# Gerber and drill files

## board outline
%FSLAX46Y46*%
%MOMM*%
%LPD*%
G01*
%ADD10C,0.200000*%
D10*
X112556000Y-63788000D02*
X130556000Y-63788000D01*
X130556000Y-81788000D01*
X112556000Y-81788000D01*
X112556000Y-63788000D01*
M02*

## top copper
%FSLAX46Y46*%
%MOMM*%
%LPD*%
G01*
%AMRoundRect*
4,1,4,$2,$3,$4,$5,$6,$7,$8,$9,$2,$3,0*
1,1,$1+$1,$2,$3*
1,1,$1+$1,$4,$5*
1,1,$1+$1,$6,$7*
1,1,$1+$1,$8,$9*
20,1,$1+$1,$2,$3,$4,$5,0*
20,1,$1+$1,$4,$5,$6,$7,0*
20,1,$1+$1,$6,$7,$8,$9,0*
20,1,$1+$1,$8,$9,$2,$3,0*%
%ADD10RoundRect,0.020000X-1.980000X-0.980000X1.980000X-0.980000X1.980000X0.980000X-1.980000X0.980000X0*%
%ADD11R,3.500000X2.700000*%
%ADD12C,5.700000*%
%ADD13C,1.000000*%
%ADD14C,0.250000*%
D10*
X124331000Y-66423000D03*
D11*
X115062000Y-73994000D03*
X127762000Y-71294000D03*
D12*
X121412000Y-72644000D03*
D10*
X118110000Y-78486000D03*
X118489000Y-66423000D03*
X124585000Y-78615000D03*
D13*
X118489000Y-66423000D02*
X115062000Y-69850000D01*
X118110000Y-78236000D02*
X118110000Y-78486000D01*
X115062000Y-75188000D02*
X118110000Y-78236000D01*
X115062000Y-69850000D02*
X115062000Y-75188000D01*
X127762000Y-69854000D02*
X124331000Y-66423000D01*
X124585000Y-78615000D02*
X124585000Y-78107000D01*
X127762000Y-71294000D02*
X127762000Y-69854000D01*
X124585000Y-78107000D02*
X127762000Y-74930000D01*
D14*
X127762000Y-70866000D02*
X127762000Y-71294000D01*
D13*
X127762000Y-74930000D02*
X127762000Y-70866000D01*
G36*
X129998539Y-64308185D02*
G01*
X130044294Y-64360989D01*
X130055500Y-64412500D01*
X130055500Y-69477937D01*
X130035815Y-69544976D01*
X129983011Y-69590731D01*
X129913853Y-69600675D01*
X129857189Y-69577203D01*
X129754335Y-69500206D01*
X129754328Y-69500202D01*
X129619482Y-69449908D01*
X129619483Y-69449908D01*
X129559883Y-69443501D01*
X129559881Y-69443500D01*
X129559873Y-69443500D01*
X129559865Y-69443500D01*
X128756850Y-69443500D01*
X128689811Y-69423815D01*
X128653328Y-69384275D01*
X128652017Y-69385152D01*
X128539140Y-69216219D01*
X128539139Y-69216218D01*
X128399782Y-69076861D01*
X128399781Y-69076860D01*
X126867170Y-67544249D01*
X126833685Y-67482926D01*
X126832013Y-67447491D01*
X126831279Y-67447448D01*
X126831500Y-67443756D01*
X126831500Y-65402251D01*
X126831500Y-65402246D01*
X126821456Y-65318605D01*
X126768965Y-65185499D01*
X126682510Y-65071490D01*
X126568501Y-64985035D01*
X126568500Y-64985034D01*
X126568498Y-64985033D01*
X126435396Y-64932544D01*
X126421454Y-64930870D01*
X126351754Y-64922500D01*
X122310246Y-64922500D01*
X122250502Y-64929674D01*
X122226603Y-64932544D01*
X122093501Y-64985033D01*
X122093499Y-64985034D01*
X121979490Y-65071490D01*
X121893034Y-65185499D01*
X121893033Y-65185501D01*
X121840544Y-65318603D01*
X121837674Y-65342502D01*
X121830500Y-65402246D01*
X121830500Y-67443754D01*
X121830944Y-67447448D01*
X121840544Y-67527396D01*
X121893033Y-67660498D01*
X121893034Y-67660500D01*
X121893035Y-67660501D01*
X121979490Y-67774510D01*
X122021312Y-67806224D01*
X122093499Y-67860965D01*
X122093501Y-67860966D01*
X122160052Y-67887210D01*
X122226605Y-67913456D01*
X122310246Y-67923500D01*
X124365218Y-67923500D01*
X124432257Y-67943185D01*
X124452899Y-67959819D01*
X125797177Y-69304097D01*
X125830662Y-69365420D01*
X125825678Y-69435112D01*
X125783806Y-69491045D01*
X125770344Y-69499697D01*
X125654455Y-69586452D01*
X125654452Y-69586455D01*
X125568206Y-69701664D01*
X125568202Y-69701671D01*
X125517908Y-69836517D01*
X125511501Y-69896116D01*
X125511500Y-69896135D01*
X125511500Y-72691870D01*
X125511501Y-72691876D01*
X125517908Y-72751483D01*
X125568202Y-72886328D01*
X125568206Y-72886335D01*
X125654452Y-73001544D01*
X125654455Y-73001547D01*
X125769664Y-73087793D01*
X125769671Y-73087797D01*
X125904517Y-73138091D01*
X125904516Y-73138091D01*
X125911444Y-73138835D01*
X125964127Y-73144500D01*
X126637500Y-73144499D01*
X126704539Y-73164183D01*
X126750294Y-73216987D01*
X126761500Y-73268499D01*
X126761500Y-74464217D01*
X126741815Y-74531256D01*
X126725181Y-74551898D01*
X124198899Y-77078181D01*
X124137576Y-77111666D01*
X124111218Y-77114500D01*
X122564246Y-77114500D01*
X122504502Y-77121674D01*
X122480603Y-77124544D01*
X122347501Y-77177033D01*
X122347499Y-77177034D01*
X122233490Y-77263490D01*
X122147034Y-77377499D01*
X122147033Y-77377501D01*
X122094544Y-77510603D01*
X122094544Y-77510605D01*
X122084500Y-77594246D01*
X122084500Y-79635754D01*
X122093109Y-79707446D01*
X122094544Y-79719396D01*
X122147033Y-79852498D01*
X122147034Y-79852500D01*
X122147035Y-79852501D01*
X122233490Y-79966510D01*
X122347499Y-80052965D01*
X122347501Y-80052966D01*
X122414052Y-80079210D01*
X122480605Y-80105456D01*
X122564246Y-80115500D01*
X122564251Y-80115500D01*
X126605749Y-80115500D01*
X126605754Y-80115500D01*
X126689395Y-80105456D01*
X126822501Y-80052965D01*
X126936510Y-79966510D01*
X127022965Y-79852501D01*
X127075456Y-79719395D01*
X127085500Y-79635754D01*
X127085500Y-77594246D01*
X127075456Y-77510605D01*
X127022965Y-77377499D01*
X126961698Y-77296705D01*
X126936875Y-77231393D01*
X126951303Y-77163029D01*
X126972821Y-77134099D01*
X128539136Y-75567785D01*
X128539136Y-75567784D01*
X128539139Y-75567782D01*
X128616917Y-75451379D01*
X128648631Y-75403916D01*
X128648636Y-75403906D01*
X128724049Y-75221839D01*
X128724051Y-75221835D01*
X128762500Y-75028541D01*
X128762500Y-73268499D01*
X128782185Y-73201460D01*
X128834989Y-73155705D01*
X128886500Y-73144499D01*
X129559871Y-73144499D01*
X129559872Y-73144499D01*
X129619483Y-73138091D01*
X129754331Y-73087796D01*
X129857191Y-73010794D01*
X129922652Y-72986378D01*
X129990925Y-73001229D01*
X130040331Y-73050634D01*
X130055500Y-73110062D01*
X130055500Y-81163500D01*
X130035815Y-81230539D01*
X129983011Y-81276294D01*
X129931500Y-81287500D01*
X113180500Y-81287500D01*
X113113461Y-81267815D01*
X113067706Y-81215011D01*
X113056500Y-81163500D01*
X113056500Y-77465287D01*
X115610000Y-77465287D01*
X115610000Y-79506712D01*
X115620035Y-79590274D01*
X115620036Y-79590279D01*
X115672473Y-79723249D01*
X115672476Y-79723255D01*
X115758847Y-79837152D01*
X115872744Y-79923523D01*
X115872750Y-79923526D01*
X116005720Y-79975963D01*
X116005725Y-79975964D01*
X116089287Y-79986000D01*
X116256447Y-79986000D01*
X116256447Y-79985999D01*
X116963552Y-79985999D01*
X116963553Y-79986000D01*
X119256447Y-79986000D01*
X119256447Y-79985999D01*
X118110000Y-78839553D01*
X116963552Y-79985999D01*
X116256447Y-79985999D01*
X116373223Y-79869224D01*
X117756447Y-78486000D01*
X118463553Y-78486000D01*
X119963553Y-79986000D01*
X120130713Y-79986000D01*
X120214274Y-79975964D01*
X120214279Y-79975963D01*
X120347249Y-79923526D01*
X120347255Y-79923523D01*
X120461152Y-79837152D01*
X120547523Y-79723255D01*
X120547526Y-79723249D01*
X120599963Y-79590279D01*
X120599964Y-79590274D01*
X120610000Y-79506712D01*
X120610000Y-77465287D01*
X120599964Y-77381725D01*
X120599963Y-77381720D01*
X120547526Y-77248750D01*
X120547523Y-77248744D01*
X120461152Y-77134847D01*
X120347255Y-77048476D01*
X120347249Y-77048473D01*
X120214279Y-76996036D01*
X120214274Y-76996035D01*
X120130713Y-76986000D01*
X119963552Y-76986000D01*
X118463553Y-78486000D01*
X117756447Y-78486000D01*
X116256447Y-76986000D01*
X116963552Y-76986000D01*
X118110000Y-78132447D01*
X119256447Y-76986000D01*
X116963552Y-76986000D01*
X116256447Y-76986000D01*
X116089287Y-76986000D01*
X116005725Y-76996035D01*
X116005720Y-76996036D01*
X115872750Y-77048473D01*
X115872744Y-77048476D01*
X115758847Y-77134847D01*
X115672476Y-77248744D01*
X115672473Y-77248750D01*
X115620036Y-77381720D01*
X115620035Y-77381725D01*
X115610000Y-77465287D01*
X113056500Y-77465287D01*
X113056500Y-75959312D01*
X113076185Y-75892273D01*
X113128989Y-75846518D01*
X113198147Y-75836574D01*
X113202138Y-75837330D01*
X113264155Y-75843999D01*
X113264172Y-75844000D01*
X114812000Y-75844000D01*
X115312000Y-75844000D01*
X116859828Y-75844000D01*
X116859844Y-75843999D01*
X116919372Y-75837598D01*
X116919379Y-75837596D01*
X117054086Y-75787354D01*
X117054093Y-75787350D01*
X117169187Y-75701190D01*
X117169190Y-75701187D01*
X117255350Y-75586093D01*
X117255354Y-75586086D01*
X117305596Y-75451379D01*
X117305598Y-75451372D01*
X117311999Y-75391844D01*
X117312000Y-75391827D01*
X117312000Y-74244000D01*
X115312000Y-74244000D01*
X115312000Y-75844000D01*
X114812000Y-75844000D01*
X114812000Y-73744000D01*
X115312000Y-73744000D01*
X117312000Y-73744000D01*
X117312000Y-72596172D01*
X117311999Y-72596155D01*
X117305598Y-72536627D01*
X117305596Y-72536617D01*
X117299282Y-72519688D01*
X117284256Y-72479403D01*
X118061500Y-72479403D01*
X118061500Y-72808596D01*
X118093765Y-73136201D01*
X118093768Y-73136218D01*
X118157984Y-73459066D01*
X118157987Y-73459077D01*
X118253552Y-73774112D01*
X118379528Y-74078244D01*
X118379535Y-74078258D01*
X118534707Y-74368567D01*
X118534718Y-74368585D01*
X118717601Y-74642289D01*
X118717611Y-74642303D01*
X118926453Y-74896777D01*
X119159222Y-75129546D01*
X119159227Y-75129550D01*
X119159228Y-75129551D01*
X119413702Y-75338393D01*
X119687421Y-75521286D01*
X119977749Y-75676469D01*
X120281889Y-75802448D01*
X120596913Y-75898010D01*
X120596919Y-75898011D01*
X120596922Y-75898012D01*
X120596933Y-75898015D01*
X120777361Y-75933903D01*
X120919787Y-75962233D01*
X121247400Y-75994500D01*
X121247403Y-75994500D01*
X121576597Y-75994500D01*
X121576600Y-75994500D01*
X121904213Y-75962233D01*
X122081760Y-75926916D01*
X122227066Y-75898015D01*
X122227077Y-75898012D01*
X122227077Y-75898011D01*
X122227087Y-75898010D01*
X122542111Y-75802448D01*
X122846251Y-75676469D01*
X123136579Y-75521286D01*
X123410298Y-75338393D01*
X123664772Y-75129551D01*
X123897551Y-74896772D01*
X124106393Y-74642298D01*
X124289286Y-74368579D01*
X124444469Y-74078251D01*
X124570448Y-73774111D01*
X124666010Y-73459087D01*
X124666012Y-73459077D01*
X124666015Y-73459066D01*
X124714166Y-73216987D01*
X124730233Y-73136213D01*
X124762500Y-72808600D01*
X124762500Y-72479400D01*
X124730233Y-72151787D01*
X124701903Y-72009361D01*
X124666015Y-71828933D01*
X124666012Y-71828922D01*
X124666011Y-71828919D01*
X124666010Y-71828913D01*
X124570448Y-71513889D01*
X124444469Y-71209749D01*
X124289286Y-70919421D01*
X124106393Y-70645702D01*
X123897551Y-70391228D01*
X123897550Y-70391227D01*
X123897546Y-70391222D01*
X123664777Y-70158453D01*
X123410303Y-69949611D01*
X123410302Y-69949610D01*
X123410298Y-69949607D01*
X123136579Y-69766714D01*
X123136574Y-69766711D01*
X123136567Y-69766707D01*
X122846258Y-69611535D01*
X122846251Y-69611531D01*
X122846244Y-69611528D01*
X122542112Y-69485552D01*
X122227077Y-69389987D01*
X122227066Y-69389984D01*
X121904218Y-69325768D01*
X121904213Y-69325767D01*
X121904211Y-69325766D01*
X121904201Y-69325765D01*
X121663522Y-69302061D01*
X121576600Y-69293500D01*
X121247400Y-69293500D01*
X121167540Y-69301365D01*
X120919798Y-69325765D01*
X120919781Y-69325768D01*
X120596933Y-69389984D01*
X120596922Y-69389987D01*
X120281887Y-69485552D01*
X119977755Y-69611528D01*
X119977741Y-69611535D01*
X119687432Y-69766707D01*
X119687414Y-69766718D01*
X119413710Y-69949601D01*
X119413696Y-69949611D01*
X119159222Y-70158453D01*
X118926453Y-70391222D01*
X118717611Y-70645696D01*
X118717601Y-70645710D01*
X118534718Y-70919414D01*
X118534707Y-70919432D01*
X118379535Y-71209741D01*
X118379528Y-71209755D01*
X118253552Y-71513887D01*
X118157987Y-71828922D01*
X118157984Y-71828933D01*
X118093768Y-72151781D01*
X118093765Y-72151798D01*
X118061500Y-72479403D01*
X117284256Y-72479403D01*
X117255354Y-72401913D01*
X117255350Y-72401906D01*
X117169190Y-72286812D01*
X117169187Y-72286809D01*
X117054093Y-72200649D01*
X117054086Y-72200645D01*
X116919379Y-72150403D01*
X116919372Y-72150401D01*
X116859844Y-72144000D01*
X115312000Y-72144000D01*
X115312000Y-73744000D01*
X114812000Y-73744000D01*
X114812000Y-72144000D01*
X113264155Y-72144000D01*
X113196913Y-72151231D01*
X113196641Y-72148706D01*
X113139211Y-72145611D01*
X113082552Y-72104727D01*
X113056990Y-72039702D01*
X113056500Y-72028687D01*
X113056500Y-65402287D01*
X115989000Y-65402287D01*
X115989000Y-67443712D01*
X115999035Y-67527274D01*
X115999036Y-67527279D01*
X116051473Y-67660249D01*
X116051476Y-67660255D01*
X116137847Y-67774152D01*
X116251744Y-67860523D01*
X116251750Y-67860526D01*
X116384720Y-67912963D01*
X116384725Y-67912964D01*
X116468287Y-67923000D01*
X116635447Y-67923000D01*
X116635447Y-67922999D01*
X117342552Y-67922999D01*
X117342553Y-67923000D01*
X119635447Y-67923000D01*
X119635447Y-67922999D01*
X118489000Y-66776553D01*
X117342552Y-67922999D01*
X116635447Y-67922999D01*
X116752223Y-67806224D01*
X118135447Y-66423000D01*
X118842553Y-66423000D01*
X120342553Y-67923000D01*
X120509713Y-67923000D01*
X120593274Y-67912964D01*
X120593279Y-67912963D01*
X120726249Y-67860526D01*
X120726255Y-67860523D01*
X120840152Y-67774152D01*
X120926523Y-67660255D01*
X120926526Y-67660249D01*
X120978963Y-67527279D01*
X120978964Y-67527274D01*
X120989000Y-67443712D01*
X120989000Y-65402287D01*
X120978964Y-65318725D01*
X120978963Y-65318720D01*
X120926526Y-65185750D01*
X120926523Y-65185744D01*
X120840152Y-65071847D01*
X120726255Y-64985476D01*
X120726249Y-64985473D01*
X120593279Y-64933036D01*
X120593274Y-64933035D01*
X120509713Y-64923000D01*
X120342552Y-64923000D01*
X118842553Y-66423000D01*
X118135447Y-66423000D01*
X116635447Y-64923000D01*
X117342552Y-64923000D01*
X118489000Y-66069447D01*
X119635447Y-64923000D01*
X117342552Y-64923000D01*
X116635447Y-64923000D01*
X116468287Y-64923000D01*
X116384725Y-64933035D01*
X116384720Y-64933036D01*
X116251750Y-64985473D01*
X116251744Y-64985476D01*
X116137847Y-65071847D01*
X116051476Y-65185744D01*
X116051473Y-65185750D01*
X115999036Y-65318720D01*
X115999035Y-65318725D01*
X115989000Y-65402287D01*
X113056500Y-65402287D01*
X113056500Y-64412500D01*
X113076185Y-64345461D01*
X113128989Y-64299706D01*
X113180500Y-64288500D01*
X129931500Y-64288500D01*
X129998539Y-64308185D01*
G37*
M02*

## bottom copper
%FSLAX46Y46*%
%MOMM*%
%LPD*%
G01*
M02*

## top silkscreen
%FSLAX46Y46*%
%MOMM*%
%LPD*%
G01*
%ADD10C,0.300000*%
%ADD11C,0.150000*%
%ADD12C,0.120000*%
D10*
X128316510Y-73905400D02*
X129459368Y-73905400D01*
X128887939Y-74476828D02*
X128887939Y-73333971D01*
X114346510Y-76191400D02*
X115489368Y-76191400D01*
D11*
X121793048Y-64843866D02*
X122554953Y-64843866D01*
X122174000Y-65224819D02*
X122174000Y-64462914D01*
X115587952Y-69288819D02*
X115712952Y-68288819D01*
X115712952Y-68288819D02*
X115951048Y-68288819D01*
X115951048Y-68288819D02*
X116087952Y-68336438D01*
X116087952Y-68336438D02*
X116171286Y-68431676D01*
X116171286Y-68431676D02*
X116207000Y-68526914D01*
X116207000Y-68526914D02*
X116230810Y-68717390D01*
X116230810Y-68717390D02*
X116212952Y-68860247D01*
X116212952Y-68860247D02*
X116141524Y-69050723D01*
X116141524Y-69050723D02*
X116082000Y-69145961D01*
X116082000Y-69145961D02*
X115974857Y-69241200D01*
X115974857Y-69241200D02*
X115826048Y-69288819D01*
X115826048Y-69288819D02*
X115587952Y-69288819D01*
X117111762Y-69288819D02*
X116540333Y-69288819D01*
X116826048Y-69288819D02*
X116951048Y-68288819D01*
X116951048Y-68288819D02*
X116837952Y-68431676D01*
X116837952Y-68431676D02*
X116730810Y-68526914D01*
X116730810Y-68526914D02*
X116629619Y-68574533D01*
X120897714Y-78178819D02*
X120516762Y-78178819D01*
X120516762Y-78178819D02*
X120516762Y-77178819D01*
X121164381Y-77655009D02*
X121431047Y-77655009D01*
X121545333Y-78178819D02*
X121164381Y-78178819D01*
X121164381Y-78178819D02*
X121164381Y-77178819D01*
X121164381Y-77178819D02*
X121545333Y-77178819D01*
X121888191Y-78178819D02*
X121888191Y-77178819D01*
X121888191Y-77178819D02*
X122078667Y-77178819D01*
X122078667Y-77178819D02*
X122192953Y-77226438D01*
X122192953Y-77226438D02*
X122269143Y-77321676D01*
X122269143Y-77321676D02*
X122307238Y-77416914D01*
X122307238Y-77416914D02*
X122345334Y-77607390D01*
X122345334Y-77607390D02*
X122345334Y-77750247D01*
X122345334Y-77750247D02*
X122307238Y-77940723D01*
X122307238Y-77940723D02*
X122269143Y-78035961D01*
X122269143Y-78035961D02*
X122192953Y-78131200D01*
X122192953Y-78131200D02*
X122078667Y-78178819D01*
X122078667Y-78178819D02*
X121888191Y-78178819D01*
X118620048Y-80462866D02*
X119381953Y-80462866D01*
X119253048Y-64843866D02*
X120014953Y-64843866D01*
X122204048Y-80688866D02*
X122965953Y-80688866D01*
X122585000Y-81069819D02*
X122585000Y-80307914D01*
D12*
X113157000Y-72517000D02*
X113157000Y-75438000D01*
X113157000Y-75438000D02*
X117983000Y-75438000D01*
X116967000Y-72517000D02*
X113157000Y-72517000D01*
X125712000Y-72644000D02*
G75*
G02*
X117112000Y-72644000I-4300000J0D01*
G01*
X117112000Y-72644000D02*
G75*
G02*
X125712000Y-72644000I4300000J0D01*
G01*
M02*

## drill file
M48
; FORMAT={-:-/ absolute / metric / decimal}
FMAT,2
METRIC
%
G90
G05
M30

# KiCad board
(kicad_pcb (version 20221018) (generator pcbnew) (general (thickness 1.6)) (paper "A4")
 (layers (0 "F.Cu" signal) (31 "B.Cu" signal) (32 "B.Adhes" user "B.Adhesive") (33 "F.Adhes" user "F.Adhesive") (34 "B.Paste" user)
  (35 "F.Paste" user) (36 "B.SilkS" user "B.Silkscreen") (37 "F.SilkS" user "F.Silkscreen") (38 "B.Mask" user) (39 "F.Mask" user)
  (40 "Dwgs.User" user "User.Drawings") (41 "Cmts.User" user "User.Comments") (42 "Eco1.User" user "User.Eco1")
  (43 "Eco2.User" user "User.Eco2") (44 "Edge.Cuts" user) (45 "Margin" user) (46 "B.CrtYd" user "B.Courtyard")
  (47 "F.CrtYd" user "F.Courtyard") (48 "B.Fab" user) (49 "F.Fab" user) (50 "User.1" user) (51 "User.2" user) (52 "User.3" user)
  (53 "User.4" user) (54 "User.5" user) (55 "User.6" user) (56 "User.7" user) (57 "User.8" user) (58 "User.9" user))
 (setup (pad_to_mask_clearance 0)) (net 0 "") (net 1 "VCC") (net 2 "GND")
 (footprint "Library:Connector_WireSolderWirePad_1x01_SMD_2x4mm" (layer "F.Cu") (at 122.331 67.423)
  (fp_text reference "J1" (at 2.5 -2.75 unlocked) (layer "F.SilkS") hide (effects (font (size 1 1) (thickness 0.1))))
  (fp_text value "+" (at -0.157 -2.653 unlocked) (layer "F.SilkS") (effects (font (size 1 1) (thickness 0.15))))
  (pad "1" smd roundrect (at 2 -1) (size 4 2) (layers "F.Cu" "F.Paste" "F.Mask") (roundrect_rratio 0.01) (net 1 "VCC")
   (thermal_bridge_angle 45)))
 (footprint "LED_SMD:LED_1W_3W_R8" (layer "F.Cu") (at 121.412 72.644)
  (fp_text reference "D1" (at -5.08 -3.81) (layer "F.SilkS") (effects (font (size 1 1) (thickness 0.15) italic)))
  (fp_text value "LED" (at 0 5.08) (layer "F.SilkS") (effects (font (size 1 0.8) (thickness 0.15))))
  (fp_line (start -8.255 -0.127) (end -8.255 2.794) (stroke (width 0.12) (type solid)) (layer "F.SilkS"))
  (fp_line (start -8.255 2.794) (end -3.429 2.794) (stroke (width 0.12) (type solid)) (layer "F.SilkS"))
  (fp_line (start -4.445 -0.127) (end -8.255 -0.127) (stroke (width 0.12) (type solid)) (layer "F.SilkS"))
  (fp_circle (center 0 0) (end -4.3 0) (stroke (width 0.12) (type solid)) (fill none) (layer "F.SilkS"))
  (pad "1" smd rect (at -6.35 1.35) (size 3.5 2.7) (layers "F.Cu" "F.Paste" "F.Mask") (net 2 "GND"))
  (pad "2" smd rect (at 6.35 -1.35) (size 3.5 2.7) (layers "F.Cu" "F.Paste" "F.Mask") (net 1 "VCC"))
  (pad "3" smd circle (at 0 0) (size 5.7 5.7) (layers "F.Cu" "F.Paste" "F.Mask")))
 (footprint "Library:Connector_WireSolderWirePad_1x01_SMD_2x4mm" (layer "F.Cu") (at 116.11 79.486)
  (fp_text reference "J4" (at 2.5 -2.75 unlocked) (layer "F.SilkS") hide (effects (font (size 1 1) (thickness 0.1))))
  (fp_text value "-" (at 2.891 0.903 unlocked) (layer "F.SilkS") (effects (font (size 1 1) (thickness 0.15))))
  (pad "1" smd roundrect (at 2 -1) (size 4 2) (layers "F.Cu" "F.Paste" "F.Mask") (roundrect_rratio 0.01) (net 2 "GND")
   (thermal_bridge_angle 45)))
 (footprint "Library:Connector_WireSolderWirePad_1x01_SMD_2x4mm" (layer "F.Cu") (at 116.489 67.423)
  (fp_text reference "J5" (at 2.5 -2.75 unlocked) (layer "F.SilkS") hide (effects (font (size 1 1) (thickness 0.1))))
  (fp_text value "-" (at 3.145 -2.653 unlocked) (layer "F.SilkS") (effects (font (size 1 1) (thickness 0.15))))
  (pad "1" smd roundrect (at 2 -1) (size 4 2) (layers "F.Cu" "F.Paste" "F.Mask") (roundrect_rratio 0.01) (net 2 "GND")
   (thermal_bridge_angle 45)))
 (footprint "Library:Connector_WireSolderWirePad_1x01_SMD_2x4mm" (layer "F.Cu") (at 122.585 79.615)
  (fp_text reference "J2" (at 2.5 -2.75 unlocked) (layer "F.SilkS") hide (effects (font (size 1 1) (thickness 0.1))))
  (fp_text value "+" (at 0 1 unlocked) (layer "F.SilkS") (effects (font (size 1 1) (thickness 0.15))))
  (pad "1" smd roundrect (at 2 -1) (size 4 2) (layers "F.Cu" "F.Paste" "F.Mask") (roundrect_rratio 0.01) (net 1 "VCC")
   (thermal_bridge_angle 45)))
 (gr_rect (start 112.556 63.788) (end 130.556 81.788) (stroke (width 0.2) (type default)) (fill none) (layer "Edge.Cuts"))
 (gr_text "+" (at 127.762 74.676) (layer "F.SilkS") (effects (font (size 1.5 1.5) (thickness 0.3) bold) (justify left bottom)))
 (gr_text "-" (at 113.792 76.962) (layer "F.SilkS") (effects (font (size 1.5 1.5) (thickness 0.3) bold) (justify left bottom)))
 (segment (start 118.489 66.423) (end 115.062 69.85) (width 1) (layer "F.Cu") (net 2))
 (segment (start 118.11 78.236) (end 118.11 78.486) (width 1) (layer "F.Cu") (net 2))
 (segment (start 115.062 75.188) (end 118.11 78.236) (width 1) (layer "F.Cu") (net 2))
 (segment (start 115.062 69.85) (end 115.062 75.188) (width 1) (layer "F.Cu") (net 2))
 (segment (start 127.762 69.854) (end 124.331 66.423) (width 1) (layer "F.Cu") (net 1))
 (segment (start 124.585 78.615) (end 124.585 78.107) (width 1) (layer "F.Cu") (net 1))
 (segment (start 127.762 71.294) (end 127.762 69.854) (width 1) (layer "F.Cu") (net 1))
 (segment (start 124.585 78.107) (end 127.762 74.93) (width 1) (layer "F.Cu") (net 1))
 (segment (start 127.762 70.866) (end 127.762 71.294) (width 0.25) (layer "F.Cu") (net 1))
 (segment (start 127.762 74.93) (end 127.762 70.866) (width 1) (layer "F.Cu") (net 1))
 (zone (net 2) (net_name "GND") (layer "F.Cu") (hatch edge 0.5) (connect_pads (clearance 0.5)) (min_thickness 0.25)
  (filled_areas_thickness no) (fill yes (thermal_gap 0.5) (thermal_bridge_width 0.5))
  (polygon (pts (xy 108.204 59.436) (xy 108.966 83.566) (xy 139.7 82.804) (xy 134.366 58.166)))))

